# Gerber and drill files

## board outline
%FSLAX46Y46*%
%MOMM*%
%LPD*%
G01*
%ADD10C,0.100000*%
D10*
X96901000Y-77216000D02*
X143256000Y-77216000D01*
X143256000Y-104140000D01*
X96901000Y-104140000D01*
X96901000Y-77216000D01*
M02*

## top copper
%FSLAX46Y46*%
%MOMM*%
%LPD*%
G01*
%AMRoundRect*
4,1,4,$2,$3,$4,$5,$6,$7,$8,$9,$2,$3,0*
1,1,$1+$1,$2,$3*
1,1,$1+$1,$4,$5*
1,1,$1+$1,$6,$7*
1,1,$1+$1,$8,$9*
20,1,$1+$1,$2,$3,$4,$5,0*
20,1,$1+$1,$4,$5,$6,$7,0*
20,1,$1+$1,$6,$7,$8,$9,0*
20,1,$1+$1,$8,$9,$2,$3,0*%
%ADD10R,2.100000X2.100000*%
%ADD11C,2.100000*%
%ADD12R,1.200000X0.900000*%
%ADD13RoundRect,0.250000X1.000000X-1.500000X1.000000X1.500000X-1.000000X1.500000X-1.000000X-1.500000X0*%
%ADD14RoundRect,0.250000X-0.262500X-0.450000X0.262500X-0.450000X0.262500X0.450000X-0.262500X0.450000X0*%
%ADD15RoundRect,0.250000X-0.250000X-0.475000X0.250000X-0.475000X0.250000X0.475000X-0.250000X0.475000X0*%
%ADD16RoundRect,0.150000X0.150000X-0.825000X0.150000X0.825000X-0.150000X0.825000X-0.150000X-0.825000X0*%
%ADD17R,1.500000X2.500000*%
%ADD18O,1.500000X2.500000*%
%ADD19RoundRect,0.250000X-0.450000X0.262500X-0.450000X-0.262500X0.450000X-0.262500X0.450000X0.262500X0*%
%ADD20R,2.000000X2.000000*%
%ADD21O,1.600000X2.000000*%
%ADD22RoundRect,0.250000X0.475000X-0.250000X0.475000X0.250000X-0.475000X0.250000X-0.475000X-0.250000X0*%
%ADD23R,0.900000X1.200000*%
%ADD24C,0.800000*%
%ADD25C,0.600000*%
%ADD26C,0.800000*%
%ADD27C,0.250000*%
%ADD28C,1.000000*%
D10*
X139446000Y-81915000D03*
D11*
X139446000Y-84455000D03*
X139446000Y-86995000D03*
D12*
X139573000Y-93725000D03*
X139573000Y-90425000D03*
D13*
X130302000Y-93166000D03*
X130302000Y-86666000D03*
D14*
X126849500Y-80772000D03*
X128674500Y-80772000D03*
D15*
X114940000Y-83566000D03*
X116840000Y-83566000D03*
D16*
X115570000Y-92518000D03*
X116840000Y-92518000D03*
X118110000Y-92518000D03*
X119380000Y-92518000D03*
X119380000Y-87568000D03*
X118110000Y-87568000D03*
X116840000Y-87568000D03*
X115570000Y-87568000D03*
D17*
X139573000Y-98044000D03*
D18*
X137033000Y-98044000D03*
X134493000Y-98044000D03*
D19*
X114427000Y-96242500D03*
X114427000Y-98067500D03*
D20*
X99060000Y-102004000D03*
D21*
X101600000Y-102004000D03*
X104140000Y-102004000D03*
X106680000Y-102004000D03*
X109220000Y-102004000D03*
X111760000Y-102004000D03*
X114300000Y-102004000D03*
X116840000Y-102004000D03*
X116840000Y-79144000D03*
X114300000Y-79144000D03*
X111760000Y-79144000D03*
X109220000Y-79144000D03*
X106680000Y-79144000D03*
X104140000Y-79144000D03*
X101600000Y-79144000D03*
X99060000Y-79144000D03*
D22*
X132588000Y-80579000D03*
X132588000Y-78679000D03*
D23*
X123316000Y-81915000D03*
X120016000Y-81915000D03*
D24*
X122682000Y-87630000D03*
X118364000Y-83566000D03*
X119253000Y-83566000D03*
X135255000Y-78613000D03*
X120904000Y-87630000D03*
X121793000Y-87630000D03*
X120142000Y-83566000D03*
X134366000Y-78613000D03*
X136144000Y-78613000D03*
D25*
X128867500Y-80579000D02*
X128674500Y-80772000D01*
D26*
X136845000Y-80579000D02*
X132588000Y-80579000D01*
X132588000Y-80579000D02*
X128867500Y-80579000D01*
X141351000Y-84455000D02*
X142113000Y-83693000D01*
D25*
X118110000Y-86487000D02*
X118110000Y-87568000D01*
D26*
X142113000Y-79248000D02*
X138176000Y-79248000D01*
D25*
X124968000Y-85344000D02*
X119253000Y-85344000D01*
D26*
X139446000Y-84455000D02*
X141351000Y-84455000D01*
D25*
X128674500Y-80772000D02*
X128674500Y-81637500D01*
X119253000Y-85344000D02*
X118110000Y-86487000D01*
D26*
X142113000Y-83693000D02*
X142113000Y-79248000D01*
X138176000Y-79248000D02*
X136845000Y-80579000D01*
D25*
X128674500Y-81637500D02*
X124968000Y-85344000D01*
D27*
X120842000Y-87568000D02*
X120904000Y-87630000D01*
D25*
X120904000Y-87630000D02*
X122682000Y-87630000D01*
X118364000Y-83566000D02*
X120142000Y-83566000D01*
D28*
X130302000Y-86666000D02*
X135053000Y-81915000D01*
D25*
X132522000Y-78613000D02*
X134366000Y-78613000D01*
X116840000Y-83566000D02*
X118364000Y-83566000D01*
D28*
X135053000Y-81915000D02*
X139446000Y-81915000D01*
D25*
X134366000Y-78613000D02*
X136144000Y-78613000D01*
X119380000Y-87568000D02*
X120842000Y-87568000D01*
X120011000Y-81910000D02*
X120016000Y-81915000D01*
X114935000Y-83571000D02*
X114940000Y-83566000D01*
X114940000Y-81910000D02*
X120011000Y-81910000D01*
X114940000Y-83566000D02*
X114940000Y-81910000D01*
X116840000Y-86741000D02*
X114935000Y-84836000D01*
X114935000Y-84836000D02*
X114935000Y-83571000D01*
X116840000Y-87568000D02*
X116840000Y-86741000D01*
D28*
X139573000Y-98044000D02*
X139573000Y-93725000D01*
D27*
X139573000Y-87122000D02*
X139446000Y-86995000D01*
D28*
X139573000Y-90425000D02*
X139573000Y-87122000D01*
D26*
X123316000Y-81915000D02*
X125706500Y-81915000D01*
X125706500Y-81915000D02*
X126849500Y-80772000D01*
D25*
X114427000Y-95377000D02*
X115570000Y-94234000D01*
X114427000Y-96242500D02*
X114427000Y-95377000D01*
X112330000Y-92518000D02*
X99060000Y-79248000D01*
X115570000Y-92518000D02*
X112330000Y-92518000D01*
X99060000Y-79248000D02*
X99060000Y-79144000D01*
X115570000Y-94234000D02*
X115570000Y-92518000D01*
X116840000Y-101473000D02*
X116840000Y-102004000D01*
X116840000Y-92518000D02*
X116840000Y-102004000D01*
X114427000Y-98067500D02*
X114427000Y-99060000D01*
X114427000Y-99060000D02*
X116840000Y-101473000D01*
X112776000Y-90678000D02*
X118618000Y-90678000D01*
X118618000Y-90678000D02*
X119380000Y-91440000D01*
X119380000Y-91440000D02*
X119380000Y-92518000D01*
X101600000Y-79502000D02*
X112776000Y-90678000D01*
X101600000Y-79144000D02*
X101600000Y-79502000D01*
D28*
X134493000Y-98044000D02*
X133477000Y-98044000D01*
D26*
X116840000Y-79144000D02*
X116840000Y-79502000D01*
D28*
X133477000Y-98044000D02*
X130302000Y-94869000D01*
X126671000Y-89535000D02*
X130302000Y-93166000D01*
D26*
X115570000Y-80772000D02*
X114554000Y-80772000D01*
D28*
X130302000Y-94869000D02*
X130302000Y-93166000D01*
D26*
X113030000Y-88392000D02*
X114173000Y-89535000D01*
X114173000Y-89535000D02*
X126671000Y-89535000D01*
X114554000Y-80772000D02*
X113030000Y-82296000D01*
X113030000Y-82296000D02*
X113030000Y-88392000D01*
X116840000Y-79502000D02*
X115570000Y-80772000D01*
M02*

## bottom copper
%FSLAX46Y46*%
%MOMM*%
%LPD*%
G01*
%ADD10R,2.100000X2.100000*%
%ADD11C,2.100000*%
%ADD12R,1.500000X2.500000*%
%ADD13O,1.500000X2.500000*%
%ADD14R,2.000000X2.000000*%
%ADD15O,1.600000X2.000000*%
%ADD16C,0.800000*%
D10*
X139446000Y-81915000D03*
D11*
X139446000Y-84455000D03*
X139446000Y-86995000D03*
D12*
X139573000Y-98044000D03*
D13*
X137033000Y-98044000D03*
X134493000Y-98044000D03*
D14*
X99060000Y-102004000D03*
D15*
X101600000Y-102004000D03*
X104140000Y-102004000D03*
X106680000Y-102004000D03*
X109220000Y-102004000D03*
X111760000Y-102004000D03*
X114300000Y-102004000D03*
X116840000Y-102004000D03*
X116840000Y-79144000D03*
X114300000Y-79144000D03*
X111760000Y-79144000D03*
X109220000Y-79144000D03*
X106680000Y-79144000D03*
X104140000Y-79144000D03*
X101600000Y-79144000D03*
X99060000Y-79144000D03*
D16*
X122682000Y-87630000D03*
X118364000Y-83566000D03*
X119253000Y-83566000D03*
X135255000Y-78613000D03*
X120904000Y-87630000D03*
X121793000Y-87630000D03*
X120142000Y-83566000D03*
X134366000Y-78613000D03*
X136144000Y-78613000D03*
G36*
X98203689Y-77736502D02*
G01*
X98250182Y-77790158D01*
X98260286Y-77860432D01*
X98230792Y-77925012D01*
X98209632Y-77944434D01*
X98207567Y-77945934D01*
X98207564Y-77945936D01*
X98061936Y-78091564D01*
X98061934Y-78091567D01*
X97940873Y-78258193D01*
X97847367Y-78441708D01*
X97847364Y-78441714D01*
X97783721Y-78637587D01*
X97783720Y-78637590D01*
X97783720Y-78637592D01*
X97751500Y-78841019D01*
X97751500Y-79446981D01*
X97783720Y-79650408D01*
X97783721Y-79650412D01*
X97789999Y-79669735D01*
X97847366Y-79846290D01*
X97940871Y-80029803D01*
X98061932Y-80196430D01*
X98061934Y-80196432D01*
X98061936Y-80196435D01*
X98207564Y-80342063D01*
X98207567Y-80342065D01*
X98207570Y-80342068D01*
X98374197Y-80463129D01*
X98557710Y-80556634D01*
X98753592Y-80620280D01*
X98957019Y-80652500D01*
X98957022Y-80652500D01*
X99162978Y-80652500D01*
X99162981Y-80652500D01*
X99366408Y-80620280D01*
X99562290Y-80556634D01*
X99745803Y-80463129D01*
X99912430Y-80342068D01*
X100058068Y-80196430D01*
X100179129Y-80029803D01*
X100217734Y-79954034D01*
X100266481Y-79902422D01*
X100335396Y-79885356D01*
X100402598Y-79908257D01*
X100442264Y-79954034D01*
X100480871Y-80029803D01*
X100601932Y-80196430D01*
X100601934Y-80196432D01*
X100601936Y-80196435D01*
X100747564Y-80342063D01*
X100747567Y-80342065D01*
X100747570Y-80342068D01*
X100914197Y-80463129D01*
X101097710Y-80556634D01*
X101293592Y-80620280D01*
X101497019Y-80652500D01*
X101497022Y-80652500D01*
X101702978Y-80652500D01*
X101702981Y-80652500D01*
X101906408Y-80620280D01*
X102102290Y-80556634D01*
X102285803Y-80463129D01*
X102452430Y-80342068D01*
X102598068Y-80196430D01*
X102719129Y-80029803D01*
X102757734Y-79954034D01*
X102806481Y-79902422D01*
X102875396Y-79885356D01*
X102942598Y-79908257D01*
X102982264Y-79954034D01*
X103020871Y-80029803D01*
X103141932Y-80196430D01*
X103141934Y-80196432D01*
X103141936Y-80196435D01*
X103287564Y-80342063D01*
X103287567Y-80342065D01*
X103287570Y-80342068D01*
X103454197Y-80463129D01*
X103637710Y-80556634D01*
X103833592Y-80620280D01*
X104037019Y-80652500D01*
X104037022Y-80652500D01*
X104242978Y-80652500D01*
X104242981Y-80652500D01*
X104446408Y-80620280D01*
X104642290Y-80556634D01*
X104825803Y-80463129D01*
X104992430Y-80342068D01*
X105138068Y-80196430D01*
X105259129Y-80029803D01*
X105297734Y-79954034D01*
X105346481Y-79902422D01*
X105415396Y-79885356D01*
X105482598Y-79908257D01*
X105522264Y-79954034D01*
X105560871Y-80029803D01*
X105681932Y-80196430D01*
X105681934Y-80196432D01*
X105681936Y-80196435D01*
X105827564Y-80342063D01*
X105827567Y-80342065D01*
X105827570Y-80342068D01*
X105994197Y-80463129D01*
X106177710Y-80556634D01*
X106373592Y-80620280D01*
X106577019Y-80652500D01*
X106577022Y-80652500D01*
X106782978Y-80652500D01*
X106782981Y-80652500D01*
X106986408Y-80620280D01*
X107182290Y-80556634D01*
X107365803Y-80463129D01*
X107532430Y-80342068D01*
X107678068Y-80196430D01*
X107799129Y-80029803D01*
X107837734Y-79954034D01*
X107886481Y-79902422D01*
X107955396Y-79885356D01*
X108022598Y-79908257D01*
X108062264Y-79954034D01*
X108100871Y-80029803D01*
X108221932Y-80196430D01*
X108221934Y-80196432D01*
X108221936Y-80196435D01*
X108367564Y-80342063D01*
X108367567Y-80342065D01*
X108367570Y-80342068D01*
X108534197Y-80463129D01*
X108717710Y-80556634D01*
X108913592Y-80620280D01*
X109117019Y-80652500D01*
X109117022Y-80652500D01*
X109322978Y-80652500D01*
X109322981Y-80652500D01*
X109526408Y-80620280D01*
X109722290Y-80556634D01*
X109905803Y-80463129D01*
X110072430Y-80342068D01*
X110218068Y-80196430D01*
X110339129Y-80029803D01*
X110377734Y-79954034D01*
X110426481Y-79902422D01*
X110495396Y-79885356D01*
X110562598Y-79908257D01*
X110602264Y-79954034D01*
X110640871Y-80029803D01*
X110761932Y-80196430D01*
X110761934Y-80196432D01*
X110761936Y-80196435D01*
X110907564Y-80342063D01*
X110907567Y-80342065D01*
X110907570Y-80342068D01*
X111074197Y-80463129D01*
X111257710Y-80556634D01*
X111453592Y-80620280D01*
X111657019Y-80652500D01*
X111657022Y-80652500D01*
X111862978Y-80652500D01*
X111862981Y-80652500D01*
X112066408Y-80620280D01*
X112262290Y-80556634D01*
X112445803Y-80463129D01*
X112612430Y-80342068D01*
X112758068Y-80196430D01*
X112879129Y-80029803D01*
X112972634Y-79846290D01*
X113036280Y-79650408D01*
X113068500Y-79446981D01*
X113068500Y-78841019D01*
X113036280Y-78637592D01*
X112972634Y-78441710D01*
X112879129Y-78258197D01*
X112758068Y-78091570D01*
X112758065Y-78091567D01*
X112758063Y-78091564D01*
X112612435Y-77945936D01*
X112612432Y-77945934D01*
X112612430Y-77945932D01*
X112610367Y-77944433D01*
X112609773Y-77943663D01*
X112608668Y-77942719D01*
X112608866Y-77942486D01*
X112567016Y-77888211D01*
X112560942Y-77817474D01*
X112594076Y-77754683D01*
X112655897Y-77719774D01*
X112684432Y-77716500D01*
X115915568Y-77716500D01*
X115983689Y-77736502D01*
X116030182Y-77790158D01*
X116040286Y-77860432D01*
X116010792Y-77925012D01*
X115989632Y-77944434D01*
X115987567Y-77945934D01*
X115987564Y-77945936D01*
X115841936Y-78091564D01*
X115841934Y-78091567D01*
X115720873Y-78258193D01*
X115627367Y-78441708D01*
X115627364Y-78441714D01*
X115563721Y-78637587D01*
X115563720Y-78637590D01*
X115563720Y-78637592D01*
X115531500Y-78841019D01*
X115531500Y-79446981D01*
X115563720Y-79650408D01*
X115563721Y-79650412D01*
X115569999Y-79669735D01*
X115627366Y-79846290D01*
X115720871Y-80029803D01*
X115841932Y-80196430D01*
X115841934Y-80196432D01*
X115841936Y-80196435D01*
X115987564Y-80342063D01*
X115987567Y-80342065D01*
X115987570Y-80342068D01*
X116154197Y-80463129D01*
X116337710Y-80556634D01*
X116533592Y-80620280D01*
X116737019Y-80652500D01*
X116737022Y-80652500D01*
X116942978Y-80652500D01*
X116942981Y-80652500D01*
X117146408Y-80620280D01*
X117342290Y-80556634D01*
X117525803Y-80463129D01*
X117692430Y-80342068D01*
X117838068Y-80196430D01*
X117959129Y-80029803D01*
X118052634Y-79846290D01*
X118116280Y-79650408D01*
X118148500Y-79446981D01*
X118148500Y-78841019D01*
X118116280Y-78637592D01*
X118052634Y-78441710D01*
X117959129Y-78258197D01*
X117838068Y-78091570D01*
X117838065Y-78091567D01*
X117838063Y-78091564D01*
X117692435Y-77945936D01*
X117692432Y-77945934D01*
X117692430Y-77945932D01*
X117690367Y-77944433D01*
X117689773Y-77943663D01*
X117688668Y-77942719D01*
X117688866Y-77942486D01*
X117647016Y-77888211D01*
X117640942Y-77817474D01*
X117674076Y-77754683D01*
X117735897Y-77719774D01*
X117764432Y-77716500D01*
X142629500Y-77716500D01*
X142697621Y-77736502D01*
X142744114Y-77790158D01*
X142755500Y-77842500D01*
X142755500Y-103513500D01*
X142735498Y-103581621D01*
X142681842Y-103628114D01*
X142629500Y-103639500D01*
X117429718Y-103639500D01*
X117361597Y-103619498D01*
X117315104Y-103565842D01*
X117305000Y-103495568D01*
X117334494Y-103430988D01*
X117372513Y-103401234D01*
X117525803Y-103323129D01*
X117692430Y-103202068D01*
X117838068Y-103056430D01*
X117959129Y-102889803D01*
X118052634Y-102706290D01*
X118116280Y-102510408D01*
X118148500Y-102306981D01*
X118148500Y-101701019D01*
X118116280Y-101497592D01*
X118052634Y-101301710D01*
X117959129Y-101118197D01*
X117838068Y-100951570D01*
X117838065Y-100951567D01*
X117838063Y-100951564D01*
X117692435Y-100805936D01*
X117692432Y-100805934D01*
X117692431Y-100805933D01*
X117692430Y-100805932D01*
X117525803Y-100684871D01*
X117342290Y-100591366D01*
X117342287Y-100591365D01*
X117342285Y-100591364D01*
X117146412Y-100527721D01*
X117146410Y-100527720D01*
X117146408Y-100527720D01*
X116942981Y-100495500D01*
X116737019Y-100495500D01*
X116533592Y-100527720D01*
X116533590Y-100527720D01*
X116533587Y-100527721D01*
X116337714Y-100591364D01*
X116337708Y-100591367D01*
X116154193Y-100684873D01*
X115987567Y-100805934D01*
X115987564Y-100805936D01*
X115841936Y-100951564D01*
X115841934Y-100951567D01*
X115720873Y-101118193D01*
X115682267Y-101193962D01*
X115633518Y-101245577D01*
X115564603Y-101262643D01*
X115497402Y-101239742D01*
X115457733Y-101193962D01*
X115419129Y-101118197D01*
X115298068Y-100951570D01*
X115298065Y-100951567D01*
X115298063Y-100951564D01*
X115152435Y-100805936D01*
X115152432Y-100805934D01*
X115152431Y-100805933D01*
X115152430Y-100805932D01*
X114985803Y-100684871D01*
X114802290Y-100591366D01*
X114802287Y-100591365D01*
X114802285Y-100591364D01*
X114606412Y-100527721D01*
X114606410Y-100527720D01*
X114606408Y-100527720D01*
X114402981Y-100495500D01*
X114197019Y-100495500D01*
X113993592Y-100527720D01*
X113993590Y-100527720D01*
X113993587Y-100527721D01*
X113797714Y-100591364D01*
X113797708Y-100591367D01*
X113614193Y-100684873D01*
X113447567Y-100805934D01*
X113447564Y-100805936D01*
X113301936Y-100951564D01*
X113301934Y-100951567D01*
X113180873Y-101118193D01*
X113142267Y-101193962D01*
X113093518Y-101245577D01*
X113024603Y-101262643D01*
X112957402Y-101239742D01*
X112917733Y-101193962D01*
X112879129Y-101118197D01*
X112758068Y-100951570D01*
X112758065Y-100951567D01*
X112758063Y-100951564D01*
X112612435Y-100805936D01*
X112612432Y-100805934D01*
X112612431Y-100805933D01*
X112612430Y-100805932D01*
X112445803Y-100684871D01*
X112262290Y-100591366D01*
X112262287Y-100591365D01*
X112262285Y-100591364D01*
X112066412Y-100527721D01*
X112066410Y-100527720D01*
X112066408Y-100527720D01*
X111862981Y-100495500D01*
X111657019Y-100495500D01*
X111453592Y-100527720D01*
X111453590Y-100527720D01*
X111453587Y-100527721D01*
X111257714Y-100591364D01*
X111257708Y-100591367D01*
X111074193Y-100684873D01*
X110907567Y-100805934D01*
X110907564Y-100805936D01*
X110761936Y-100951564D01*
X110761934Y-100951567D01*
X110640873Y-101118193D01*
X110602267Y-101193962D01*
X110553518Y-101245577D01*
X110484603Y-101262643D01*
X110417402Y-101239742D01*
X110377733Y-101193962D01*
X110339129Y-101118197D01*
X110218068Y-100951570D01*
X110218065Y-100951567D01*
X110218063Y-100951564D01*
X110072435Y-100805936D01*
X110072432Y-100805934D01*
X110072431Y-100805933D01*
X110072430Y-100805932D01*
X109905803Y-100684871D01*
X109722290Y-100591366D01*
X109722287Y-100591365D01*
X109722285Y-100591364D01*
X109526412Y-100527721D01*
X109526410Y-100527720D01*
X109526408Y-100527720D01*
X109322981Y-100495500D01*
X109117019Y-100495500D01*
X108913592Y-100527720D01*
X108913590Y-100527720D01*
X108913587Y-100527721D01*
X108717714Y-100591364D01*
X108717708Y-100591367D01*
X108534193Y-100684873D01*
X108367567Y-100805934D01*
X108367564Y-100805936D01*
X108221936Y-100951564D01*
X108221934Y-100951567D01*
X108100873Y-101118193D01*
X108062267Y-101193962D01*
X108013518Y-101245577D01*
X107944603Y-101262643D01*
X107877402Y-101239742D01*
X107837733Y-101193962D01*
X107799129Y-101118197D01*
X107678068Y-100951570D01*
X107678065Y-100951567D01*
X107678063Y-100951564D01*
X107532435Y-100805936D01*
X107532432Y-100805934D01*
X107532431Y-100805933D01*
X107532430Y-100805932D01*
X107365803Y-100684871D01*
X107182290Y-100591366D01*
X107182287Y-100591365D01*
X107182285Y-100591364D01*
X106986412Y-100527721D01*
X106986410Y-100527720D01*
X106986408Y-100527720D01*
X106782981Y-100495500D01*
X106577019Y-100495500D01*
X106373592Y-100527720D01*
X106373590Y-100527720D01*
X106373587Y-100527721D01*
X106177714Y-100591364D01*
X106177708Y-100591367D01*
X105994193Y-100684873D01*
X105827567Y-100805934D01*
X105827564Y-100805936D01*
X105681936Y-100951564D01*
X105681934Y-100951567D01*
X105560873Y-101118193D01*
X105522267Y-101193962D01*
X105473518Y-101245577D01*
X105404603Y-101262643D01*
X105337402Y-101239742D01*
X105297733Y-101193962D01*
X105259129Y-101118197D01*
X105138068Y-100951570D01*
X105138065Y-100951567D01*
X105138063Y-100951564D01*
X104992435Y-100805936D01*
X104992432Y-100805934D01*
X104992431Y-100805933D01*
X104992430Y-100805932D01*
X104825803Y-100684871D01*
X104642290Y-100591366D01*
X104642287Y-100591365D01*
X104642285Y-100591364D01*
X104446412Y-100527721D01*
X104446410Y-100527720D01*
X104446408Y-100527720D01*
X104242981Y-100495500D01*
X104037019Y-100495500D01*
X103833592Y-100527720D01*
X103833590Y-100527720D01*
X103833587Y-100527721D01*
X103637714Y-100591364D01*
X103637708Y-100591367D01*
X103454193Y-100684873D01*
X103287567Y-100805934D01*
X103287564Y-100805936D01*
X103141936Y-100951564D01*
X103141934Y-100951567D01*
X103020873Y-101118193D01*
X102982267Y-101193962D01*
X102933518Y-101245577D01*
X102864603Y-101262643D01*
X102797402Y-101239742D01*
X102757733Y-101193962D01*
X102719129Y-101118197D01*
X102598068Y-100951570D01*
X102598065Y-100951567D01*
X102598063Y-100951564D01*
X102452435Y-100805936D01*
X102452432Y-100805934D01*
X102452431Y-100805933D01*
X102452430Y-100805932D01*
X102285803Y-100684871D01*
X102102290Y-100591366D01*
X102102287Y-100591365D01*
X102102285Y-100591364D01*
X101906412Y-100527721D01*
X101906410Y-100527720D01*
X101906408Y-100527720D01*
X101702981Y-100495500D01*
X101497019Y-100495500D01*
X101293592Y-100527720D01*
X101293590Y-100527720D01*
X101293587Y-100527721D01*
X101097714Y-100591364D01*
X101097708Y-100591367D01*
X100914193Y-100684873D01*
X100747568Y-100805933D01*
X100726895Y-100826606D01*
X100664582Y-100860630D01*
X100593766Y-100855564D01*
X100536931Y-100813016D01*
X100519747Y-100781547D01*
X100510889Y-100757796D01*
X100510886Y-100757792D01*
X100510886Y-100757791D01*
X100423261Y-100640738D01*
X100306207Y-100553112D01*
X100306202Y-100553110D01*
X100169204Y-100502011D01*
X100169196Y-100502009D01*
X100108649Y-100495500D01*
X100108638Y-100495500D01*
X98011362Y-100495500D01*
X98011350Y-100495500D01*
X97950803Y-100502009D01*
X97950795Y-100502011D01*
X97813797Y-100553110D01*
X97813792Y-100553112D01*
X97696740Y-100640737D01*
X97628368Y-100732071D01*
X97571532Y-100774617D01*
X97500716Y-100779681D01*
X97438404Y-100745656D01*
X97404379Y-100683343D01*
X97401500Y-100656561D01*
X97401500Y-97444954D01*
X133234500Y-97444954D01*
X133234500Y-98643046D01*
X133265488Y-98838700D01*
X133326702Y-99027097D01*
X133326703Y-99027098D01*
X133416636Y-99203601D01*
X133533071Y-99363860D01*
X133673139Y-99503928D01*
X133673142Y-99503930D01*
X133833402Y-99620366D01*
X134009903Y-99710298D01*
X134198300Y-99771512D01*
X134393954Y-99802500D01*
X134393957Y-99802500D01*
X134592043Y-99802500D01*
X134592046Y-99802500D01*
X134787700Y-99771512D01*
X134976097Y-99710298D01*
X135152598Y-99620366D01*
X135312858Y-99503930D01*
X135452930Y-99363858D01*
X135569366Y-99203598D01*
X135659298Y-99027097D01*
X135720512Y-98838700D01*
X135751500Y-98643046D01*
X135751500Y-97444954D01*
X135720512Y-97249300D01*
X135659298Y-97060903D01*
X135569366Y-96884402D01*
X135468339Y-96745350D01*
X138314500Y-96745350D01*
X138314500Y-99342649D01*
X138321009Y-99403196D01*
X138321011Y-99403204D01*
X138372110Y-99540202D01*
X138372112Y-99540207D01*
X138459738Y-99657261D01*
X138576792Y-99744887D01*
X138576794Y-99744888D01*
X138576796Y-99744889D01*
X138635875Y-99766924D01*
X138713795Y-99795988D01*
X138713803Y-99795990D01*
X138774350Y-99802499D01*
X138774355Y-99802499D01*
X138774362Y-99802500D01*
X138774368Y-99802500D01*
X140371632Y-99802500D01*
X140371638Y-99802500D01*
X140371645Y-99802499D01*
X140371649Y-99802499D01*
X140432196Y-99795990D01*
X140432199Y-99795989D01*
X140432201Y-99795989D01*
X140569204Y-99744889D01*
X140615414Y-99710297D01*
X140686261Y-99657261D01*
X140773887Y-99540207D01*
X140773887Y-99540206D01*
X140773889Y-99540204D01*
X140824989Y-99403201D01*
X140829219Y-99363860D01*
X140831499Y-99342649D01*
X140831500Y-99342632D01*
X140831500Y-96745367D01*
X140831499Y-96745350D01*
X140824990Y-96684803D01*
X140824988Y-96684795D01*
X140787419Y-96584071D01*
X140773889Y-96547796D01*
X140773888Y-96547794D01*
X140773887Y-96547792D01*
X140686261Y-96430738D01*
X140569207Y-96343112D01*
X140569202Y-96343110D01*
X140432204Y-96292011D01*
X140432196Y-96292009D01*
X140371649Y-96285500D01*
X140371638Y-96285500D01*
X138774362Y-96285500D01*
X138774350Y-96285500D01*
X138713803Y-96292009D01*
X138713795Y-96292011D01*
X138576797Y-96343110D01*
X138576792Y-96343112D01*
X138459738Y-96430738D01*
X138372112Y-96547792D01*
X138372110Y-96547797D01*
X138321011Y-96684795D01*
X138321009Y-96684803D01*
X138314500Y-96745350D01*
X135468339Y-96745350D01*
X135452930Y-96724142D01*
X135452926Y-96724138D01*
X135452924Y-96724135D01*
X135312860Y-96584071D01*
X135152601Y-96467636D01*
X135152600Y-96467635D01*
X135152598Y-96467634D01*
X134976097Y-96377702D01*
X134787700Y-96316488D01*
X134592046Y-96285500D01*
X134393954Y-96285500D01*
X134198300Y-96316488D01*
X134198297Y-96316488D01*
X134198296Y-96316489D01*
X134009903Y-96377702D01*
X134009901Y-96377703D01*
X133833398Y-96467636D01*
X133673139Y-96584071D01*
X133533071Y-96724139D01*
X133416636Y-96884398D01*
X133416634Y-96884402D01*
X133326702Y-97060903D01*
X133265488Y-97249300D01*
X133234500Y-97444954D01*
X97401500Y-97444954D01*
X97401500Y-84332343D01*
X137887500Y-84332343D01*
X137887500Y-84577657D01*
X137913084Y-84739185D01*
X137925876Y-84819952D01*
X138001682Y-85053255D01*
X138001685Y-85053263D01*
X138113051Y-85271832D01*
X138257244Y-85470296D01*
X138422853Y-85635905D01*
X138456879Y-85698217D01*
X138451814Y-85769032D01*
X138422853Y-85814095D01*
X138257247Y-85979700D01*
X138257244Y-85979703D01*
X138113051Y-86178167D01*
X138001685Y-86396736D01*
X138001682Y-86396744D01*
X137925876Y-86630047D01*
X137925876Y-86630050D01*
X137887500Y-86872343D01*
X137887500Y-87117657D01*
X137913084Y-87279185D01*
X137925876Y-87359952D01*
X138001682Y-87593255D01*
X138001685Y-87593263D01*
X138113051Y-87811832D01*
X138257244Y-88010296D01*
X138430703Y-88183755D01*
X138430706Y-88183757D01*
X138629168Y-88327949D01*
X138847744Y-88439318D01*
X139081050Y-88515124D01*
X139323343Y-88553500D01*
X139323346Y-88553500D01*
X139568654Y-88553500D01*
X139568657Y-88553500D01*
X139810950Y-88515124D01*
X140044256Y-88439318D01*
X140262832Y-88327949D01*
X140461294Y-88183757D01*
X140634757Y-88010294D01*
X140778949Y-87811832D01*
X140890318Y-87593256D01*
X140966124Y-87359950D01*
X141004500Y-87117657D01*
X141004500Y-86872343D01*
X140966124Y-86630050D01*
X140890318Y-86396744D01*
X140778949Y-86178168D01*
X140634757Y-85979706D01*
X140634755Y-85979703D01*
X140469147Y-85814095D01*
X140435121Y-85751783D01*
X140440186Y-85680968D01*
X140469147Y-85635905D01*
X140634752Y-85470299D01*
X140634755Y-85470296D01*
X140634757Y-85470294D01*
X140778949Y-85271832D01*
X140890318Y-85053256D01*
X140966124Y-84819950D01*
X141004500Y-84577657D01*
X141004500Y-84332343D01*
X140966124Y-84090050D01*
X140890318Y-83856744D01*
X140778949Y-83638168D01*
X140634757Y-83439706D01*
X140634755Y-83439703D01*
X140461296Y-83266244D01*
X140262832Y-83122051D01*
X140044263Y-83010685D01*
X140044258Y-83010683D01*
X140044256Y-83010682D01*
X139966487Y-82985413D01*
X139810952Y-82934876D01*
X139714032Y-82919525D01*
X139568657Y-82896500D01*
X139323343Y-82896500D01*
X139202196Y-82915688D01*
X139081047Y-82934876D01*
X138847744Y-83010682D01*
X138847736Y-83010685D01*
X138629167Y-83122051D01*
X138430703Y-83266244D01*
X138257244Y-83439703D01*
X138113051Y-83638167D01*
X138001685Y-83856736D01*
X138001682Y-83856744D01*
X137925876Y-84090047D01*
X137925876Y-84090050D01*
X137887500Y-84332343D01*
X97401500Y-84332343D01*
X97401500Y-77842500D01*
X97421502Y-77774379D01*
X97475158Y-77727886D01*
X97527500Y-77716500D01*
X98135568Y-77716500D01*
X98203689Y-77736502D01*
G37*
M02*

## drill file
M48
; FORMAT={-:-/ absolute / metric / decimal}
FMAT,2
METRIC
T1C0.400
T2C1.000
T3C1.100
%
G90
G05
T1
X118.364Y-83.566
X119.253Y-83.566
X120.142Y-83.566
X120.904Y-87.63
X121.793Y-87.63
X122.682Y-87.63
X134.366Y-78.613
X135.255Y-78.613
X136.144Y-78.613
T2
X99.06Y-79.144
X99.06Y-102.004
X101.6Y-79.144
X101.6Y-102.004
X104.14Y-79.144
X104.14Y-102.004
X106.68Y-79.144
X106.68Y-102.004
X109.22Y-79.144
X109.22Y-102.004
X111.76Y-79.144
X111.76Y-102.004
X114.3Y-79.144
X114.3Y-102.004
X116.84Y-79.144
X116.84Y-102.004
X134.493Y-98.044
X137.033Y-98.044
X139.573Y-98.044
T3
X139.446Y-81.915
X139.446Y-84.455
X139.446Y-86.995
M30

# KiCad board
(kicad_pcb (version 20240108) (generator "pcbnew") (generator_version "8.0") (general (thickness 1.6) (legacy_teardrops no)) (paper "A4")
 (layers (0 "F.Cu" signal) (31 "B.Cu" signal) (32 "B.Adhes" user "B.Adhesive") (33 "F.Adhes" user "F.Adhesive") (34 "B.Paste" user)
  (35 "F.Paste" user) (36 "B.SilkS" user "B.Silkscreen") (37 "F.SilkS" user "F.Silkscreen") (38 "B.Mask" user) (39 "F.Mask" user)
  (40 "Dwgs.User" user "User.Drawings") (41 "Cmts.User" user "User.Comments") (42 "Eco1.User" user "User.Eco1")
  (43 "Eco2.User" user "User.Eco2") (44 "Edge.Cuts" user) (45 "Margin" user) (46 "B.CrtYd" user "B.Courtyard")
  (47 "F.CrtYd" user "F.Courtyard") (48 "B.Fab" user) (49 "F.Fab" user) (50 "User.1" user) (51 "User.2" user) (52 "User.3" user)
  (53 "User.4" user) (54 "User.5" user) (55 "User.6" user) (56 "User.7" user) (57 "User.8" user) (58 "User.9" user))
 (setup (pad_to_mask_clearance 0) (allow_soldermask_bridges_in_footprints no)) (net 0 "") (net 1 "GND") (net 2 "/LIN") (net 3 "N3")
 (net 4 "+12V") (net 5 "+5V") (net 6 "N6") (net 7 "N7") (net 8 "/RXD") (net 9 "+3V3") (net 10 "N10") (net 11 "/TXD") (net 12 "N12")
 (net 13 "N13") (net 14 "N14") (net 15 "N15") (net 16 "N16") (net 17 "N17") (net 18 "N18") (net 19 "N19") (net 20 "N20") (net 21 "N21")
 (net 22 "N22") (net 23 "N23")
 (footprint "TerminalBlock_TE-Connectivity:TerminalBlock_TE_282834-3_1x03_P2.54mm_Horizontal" (layer "F.Cu") (at 139.446 81.915 -90)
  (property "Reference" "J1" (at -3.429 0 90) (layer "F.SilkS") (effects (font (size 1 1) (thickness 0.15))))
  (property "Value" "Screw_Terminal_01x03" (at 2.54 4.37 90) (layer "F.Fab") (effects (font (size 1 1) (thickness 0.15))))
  (pad "1" thru_hole rect (at 0 0 270) (size 2.1 2.1) (drill 1.1) (layers "*.Cu" "*.Mask") (remove_unused_layers no) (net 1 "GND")
   (zone_connect 2))
  (pad "2" thru_hole circle (at 2.54 0 270) (size 2.1 2.1) (drill 1.1) (layers "*.Cu" "*.Mask") (remove_unused_layers no) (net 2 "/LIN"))
  (pad "3" thru_hole circle (at 5.08 0 270) (size 2.1 2.1) (drill 1.1) (layers "*.Cu" "*.Mask") (remove_unused_layers no) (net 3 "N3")))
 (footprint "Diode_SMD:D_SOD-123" (layer "F.Cu") (at 139.573 92.075 90)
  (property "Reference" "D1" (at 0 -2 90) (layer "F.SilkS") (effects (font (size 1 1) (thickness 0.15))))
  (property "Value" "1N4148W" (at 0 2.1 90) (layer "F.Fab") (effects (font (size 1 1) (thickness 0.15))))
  (pad "1" smd rect (at -1.65 0 90) (size 0.9 1.2) (layers "F.Cu" "F.Paste" "F.Mask") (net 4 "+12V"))
  (pad "2" smd rect (at 1.65 0 90) (size 0.9 1.2) (layers "F.Cu" "F.Paste" "F.Mask") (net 3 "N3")))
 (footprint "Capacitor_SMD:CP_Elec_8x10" (layer "F.Cu") (at 130.302 89.916 90)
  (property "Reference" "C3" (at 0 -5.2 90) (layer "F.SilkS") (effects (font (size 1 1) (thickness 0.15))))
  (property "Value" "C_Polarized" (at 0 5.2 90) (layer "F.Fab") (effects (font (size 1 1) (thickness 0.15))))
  (pad "1" smd roundrect (at -3.25 0 90) (size 3.5 2.5) (layers "F.Cu" "F.Paste" "F.Mask") (roundrect_rratio 0.1) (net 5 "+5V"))
  (pad "2" smd roundrect (at 3.25 0 90) (size 3.5 2.5) (layers "F.Cu" "F.Paste" "F.Mask") (roundrect_rratio 0.1) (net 1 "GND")))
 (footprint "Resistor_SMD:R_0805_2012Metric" (layer "F.Cu") (at 127.762 80.772)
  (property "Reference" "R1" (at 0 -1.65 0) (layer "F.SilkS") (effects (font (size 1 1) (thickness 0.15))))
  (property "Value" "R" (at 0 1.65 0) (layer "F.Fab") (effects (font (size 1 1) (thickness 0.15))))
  (pad "1" smd roundrect (at -0.9125 0) (size 1.025 1.4) (layers "F.Cu" "F.Paste" "F.Mask") (roundrect_rratio 0.243902439) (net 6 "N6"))
  (pad "2" smd roundrect (at 0.9125 0) (size 1.025 1.4) (layers "F.Cu" "F.Paste" "F.Mask") (roundrect_rratio 0.243902439) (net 2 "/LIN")))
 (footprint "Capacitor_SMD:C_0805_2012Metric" (layer "F.Cu") (at 115.89 83.566)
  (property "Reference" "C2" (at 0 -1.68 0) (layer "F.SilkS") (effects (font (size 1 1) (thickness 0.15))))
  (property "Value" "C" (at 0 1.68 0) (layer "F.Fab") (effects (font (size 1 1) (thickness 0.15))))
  (pad "1" smd roundrect (at -0.95 0) (size 1 1.45) (layers "F.Cu" "F.Paste" "F.Mask") (roundrect_rratio 0.25) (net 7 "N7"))
  (pad "2" smd roundrect (at 0.95 0) (size 1 1.45) (layers "F.Cu" "F.Paste" "F.Mask") (roundrect_rratio 0.25) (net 1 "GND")))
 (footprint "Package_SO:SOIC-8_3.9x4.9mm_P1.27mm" (layer "F.Cu") (at 117.475 90.043 90)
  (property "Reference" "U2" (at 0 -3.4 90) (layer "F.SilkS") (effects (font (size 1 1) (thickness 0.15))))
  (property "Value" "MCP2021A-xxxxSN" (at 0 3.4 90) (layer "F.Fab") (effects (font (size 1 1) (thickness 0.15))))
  (pad "1" smd roundrect (at -2.475 -1.905 90) (size 1.95 0.6) (layers "F.Cu" "F.Paste" "F.Mask") (roundrect_rratio 0.25) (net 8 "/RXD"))
  (pad "2" smd roundrect (at -2.475 -0.635 90) (size 1.95 0.6) (layers "F.Cu" "F.Paste" "F.Mask") (roundrect_rratio 0.25) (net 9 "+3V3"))
  (pad "3" smd roundrect (at -2.475 0.635 90) (size 1.95 0.6) (layers "F.Cu" "F.Paste" "F.Mask") (roundrect_rratio 0.25) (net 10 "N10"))
  (pad "4" smd roundrect (at -2.475 1.905 90) (size 1.95 0.6) (layers "F.Cu" "F.Paste" "F.Mask") (roundrect_rratio 0.25) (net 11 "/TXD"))
  (pad "5" smd roundrect (at 2.475 1.905 90) (size 1.95 0.6) (layers "F.Cu" "F.Paste" "F.Mask") (roundrect_rratio 0.25) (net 1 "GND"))
  (pad "6" smd roundrect (at 2.475 0.635 90) (size 1.95 0.6) (layers "F.Cu" "F.Paste" "F.Mask") (roundrect_rratio 0.25) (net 2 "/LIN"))
  (pad "7" smd roundrect (at 2.475 -0.635 90) (size 1.95 0.6) (layers "F.Cu" "F.Paste" "F.Mask") (roundrect_rratio 0.25) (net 7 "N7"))
  (pad "8" smd roundrect (at 2.475 -1.905 90) (size 1.95 0.6) (layers "F.Cu" "F.Paste" "F.Mask") (roundrect_rratio 0.25) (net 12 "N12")))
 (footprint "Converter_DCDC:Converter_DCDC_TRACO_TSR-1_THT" (layer "F.Cu") (at 139.573 98.044 180)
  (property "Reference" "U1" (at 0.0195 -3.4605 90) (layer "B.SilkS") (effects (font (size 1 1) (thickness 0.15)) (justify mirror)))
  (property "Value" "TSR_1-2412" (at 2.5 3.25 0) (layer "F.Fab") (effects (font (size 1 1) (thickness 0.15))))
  (pad "1" thru_hole rect (at 0 0 180) (size 1.5 2.5) (drill 1) (layers "*.Cu" "*.Mask") (remove_unused_layers no) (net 4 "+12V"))
  (pad "2" thru_hole oval (at 2.54 0 180) (size 1.5 2.5) (drill 1) (layers "*.Cu" "*.Mask") (remove_unused_layers no) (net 1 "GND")
   (zone_connect 2))
  (pad "3" thru_hole oval (at 5.08 0 180) (size 1.5 2.5) (drill 1) (layers "*.Cu" "*.Mask") (remove_unused_layers no) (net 5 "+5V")))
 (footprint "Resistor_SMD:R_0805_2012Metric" (layer "F.Cu") (at 114.427 97.155 -90)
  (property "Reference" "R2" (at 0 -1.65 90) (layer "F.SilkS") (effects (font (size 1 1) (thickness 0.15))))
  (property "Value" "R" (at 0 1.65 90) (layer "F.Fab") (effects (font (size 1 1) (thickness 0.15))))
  (pad "1" smd roundrect (at -0.9125 0 270) (size 1.025 1.4) (layers "F.Cu" "F.Paste" "F.Mask") (roundrect_rratio 0.243902439)
   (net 8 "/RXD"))
  (pad "2" smd roundrect (at 0.9125 0 270) (size 1.025 1.4) (layers "F.Cu" "F.Paste" "F.Mask") (roundrect_rratio 0.243902439) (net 9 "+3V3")))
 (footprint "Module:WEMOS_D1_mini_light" (layer "F.Cu") (at 99.06 102.004 90)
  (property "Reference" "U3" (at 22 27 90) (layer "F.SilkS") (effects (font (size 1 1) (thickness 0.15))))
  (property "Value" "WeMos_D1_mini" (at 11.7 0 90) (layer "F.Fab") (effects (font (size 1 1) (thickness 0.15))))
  (pad "1" thru_hole rect (at 0 0 90) (size 2 2) (drill 1) (layers "*.Cu" "*.Mask") (remove_unused_layers no) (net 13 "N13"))
  (pad "2" thru_hole oval (at 0 2.54 90) (size 2 1.6) (drill 1) (layers "*.Cu" "*.Mask") (remove_unused_layers no) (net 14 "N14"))
  (pad "3" thru_hole oval (at 0 5.08 90) (size 2 1.6) (drill 1) (layers "*.Cu" "*.Mask") (remove_unused_layers no) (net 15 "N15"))
  (pad "4" thru_hole oval (at 0 7.62 90) (size 2 1.6) (drill 1) (layers "*.Cu" "*.Mask") (remove_unused_layers no) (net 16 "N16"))
  (pad "5" thru_hole oval (at 0 10.16 90) (size 2 1.6) (drill 1) (layers "*.Cu" "*.Mask") (remove_unused_layers no) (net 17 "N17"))
  (pad "6" thru_hole oval (at 0 12.7 90) (size 2 1.6) (drill 1) (layers "*.Cu" "*.Mask") (remove_unused_layers no) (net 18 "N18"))
  (pad "7" thru_hole oval (at 0 15.24 90) (size 2 1.6) (drill 1) (layers "*.Cu" "*.Mask") (remove_unused_layers no) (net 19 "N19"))
  (pad "8" thru_hole oval (at 0 17.78 90) (size 2 1.6) (drill 1) (layers "*.Cu" "*.Mask") (remove_unused_layers no) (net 9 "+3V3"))
  (pad "9" thru_hole oval (at 22.86 17.78 90) (size 2 1.6) (drill 1) (layers "*.Cu" "*.Mask") (remove_unused_layers no) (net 5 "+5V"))
  (pad "10" thru_hole oval (at 22.86 15.24 90) (size 2 1.6) (drill 1) (layers "*.Cu" "*.Mask") (remove_unused_layers no) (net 1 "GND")
   (zone_connect 2))
  (pad "11" thru_hole oval (at 22.86 12.7 90) (size 2 1.6) (drill 1) (layers "*.Cu" "*.Mask") (remove_unused_layers no) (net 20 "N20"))
  (pad "12" thru_hole oval (at 22.86 10.16 90) (size 2 1.6) (drill 1) (layers "*.Cu" "*.Mask") (remove_unused_layers no) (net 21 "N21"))
  (pad "13" thru_hole oval (at 22.86 7.62 90) (size 2 1.6) (drill 1) (layers "*.Cu" "*.Mask") (remove_unused_layers no) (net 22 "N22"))
  (pad "14" thru_hole oval (at 22.86 5.08 90) (size 2 1.6) (drill 1) (layers "*.Cu" "*.Mask") (remove_unused_layers no) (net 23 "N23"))
  (pad "15" thru_hole oval (at 22.86 2.54 90) (size 2 1.6) (drill 1) (layers "*.Cu" "*.Mask") (remove_unused_layers no) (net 11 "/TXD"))
  (pad "16" thru_hole oval (at 22.86 0 90) (size 2 1.6) (drill 1) (layers "*.Cu" "*.Mask") (remove_unused_layers no) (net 8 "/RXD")))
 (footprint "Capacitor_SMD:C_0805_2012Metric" (layer "F.Cu") (at 132.588 79.629 90)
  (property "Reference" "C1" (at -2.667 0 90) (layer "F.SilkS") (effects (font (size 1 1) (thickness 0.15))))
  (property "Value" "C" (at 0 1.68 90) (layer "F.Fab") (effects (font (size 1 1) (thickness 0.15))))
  (pad "1" smd roundrect (at -0.95 0 90) (size 1 1.45) (layers "F.Cu" "F.Paste" "F.Mask") (roundrect_rratio 0.25) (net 2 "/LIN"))
  (pad "2" smd roundrect (at 0.95 0 90) (size 1 1.45) (layers "F.Cu" "F.Paste" "F.Mask") (roundrect_rratio 0.25) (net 1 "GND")))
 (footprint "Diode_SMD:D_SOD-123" (layer "F.Cu") (at 121.666 81.915 180)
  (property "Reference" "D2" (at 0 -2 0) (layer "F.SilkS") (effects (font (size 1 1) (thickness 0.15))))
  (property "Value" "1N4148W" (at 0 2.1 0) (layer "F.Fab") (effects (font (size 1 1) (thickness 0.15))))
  (pad "1" smd rect (at -1.65 0 180) (size 0.9 1.2) (layers "F.Cu" "F.Paste" "F.Mask") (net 6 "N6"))
  (pad "2" smd rect (at 1.65 0 180) (size 0.9 1.2) (layers "F.Cu" "F.Paste" "F.Mask") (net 7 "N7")))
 (gr_rect (start 96.901 77.216) (end 143.256 104.14) (stroke (width 0.1) (type solid)) (fill none) (layer "Edge.Cuts"))
 (segment (start 128.8675 80.579) (end 128.6745 80.772) (width 0.6) (layer "F.Cu") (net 2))
 (segment (start 136.845 80.579) (end 132.588 80.579) (width 0.8) (layer "F.Cu") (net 2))
 (segment (start 132.588 80.579) (end 128.8675 80.579) (width 0.8) (layer "F.Cu") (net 2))
 (segment (start 141.351 84.455) (end 142.113 83.693) (width 0.8) (layer "F.Cu") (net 2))
 (segment (start 118.11 86.487) (end 118.11 87.568) (width 0.6) (layer "F.Cu") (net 2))
 (segment (start 142.113 79.248) (end 138.176 79.248) (width 0.8) (layer "F.Cu") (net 2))
 (segment (start 124.968 85.344) (end 119.253 85.344) (width 0.6) (layer "F.Cu") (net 2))
 (segment (start 139.446 84.455) (end 141.351 84.455) (width 0.8) (layer "F.Cu") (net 2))
 (segment (start 128.6745 80.772) (end 128.6745 81.6375) (width 0.6) (layer "F.Cu") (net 2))
 (segment (start 119.253 85.344) (end 118.11 86.487) (width 0.6) (layer "F.Cu") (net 2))
 (segment (start 142.113 83.693) (end 142.113 79.248) (width 0.8) (layer "F.Cu") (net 2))
 (segment (start 138.176 79.248) (end 136.845 80.579) (width 0.8) (layer "F.Cu") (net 2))
 (segment (start 128.6745 81.6375) (end 124.968 85.344) (width 0.6) (layer "F.Cu") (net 2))
 (segment (start 120.842 87.568) (end 120.904 87.63) (width 0.25) (layer "F.Cu") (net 1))
 (segment (start 120.904 87.63) (end 122.682 87.63) (width 0.6) (layer "F.Cu") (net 1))
 (segment (start 118.364 83.566) (end 120.142 83.566) (width 0.6) (layer "F.Cu") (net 1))
 (segment (start 130.302 86.666) (end 135.053 81.915) (width 1) (layer "F.Cu") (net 1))
 (segment (start 132.522 78.613) (end 134.366 78.613) (width 0.6) (layer "F.Cu") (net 1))
 (segment (start 116.84 83.566) (end 118.364 83.566) (width 0.6) (layer "F.Cu") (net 1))
 (segment (start 135.053 81.915) (end 139.446 81.915) (width 1) (layer "F.Cu") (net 1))
 (segment (start 134.366 78.613) (end 136.144 78.613) (width 0.6) (layer "F.Cu") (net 1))
 (segment (start 119.38 87.568) (end 120.842 87.568) (width 0.6) (layer "F.Cu") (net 1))
 (via (at 122.682 87.63) (size 0.8) (drill 0.4) (layers "F.Cu" "B.Cu") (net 1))
 (via (at 118.364 83.566) (size 0.8) (drill 0.4) (layers "F.Cu" "B.Cu") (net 1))
 (via (at 119.253 83.566) (size 0.8) (drill 0.4) (layers "F.Cu" "B.Cu") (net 1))
 (via (at 135.255 78.613) (size 0.8) (drill 0.4) (layers "F.Cu" "B.Cu") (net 1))
 (via (at 120.904 87.63) (size 0.8) (drill 0.4) (layers "F.Cu" "B.Cu") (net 1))
 (via (at 121.793 87.63) (size 0.8) (drill 0.4) (layers "F.Cu" "B.Cu") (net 1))
 (via (at 120.142 83.566) (size 0.8) (drill 0.4) (layers "F.Cu" "B.Cu") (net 1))
 (via (at 134.366 78.613) (size 0.8) (drill 0.4) (layers "F.Cu" "B.Cu") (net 1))
 (via (at 136.144 78.613) (size 0.8) (drill 0.4) (layers "F.Cu" "B.Cu") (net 1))
 (segment (start 120.011 81.91) (end 120.016 81.915) (width 0.6) (layer "F.Cu") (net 7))
 (segment (start 114.935 83.571) (end 114.94 83.566) (width 0.6) (layer "F.Cu") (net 7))
 (segment (start 114.94 81.91) (end 120.011 81.91) (width 0.6) (layer "F.Cu") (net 7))
 (segment (start 114.94 83.566) (end 114.94 81.91) (width 0.6) (layer "F.Cu") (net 7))
 (segment (start 116.84 86.741) (end 114.935 84.836) (width 0.6) (layer "F.Cu") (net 7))
 (segment (start 114.935 84.836) (end 114.935 83.571) (width 0.6) (layer "F.Cu") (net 7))
 (segment (start 116.84 87.568) (end 116.84 86.741) (width 0.6) (layer "F.Cu") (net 7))
 (segment (start 139.573 98.044) (end 139.573 93.725) (width 1) (layer "F.Cu") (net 4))
 (segment (start 139.573 87.122) (end 139.446 86.995) (width 0.25) (layer "F.Cu") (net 3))
 (segment (start 139.573 90.425) (end 139.573 87.122) (width 1) (layer "F.Cu") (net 3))
 (segment (start 123.316 81.915) (end 125.7065 81.915) (width 0.8) (layer "F.Cu") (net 6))
 (segment (start 125.7065 81.915) (end 126.8495 80.772) (width 0.8) (layer "F.Cu") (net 6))
 (segment (start 114.427 95.377) (end 115.57 94.234) (width 0.6) (layer "F.Cu") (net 8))
 (segment (start 114.427 96.2425) (end 114.427 95.377) (width 0.6) (layer "F.Cu") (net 8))
 (segment (start 112.33 92.518) (end 99.06 79.248) (width 0.6) (layer "F.Cu") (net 8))
 (segment (start 115.57 92.518) (end 112.33 92.518) (width 0.6) (layer "F.Cu") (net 8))
 (segment (start 99.06 79.248) (end 99.06 79.144) (width 0.6) (layer "F.Cu") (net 8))
 (segment (start 115.57 94.234) (end 115.57 92.518) (width 0.6) (layer "F.Cu") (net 8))
 (segment (start 116.84 101.473) (end 116.84 102.004) (width 0.6) (layer "F.Cu") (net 9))
 (segment (start 116.84 92.518) (end 116.84 102.004) (width 0.6) (layer "F.Cu") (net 9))
 (segment (start 114.427 98.0675) (end 114.427 99.06) (width 0.6) (layer "F.Cu") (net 9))
 (segment (start 114.427 99.06) (end 116.84 101.473) (width 0.6) (layer "F.Cu") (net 9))
 (segment (start 112.776 90.678) (end 118.618 90.678) (width 0.6) (layer "F.Cu") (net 11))
 (segment (start 118.618 90.678) (end 119.38 91.44) (width 0.6) (layer "F.Cu") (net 11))
 (segment (start 119.38 91.44) (end 119.38 92.518) (width 0.6) (layer "F.Cu") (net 11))
 (segment (start 101.6 79.502) (end 112.776 90.678) (width 0.6) (layer "F.Cu") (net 11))
 (segment (start 101.6 79.144) (end 101.6 79.502) (width 0.6) (layer "F.Cu") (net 11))
 (segment (start 134.493 98.044) (end 133.477 98.044) (width 1) (layer "F.Cu") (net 5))
 (segment (start 116.84 79.144) (end 116.84 79.502) (width 0.8) (layer "F.Cu") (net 5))
 (segment (start 133.477 98.044) (end 130.302 94.869) (width 1) (layer "F.Cu") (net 5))
 (segment (start 126.671 89.535) (end 130.302 93.166) (width 1) (layer "F.Cu") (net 5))
 (segment (start 115.57 80.772) (end 114.554 80.772) (width 0.8) (layer "F.Cu") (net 5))
 (segment (start 130.302 94.869) (end 130.302 93.166) (width 1) (layer "F.Cu") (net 5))
 (segment (start 113.03 88.392) (end 114.173 89.535) (width 0.8) (layer "F.Cu") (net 5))
 (segment (start 114.173 89.535) (end 126.671 89.535) (width 0.8) (layer "F.Cu") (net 5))
 (segment (start 114.554 80.772) (end 113.03 82.296) (width 0.8) (layer "F.Cu") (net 5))
 (segment (start 113.03 82.296) (end 113.03 88.392) (width 0.8) (layer "F.Cu") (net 5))
 (segment (start 116.84 79.502) (end 115.57 80.772) (width 0.8) (layer "F.Cu") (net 5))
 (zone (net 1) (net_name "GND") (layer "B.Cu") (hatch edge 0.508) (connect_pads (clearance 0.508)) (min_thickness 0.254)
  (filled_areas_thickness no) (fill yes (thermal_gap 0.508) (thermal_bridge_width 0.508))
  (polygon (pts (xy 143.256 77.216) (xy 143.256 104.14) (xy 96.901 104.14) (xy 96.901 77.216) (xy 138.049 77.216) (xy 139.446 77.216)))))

